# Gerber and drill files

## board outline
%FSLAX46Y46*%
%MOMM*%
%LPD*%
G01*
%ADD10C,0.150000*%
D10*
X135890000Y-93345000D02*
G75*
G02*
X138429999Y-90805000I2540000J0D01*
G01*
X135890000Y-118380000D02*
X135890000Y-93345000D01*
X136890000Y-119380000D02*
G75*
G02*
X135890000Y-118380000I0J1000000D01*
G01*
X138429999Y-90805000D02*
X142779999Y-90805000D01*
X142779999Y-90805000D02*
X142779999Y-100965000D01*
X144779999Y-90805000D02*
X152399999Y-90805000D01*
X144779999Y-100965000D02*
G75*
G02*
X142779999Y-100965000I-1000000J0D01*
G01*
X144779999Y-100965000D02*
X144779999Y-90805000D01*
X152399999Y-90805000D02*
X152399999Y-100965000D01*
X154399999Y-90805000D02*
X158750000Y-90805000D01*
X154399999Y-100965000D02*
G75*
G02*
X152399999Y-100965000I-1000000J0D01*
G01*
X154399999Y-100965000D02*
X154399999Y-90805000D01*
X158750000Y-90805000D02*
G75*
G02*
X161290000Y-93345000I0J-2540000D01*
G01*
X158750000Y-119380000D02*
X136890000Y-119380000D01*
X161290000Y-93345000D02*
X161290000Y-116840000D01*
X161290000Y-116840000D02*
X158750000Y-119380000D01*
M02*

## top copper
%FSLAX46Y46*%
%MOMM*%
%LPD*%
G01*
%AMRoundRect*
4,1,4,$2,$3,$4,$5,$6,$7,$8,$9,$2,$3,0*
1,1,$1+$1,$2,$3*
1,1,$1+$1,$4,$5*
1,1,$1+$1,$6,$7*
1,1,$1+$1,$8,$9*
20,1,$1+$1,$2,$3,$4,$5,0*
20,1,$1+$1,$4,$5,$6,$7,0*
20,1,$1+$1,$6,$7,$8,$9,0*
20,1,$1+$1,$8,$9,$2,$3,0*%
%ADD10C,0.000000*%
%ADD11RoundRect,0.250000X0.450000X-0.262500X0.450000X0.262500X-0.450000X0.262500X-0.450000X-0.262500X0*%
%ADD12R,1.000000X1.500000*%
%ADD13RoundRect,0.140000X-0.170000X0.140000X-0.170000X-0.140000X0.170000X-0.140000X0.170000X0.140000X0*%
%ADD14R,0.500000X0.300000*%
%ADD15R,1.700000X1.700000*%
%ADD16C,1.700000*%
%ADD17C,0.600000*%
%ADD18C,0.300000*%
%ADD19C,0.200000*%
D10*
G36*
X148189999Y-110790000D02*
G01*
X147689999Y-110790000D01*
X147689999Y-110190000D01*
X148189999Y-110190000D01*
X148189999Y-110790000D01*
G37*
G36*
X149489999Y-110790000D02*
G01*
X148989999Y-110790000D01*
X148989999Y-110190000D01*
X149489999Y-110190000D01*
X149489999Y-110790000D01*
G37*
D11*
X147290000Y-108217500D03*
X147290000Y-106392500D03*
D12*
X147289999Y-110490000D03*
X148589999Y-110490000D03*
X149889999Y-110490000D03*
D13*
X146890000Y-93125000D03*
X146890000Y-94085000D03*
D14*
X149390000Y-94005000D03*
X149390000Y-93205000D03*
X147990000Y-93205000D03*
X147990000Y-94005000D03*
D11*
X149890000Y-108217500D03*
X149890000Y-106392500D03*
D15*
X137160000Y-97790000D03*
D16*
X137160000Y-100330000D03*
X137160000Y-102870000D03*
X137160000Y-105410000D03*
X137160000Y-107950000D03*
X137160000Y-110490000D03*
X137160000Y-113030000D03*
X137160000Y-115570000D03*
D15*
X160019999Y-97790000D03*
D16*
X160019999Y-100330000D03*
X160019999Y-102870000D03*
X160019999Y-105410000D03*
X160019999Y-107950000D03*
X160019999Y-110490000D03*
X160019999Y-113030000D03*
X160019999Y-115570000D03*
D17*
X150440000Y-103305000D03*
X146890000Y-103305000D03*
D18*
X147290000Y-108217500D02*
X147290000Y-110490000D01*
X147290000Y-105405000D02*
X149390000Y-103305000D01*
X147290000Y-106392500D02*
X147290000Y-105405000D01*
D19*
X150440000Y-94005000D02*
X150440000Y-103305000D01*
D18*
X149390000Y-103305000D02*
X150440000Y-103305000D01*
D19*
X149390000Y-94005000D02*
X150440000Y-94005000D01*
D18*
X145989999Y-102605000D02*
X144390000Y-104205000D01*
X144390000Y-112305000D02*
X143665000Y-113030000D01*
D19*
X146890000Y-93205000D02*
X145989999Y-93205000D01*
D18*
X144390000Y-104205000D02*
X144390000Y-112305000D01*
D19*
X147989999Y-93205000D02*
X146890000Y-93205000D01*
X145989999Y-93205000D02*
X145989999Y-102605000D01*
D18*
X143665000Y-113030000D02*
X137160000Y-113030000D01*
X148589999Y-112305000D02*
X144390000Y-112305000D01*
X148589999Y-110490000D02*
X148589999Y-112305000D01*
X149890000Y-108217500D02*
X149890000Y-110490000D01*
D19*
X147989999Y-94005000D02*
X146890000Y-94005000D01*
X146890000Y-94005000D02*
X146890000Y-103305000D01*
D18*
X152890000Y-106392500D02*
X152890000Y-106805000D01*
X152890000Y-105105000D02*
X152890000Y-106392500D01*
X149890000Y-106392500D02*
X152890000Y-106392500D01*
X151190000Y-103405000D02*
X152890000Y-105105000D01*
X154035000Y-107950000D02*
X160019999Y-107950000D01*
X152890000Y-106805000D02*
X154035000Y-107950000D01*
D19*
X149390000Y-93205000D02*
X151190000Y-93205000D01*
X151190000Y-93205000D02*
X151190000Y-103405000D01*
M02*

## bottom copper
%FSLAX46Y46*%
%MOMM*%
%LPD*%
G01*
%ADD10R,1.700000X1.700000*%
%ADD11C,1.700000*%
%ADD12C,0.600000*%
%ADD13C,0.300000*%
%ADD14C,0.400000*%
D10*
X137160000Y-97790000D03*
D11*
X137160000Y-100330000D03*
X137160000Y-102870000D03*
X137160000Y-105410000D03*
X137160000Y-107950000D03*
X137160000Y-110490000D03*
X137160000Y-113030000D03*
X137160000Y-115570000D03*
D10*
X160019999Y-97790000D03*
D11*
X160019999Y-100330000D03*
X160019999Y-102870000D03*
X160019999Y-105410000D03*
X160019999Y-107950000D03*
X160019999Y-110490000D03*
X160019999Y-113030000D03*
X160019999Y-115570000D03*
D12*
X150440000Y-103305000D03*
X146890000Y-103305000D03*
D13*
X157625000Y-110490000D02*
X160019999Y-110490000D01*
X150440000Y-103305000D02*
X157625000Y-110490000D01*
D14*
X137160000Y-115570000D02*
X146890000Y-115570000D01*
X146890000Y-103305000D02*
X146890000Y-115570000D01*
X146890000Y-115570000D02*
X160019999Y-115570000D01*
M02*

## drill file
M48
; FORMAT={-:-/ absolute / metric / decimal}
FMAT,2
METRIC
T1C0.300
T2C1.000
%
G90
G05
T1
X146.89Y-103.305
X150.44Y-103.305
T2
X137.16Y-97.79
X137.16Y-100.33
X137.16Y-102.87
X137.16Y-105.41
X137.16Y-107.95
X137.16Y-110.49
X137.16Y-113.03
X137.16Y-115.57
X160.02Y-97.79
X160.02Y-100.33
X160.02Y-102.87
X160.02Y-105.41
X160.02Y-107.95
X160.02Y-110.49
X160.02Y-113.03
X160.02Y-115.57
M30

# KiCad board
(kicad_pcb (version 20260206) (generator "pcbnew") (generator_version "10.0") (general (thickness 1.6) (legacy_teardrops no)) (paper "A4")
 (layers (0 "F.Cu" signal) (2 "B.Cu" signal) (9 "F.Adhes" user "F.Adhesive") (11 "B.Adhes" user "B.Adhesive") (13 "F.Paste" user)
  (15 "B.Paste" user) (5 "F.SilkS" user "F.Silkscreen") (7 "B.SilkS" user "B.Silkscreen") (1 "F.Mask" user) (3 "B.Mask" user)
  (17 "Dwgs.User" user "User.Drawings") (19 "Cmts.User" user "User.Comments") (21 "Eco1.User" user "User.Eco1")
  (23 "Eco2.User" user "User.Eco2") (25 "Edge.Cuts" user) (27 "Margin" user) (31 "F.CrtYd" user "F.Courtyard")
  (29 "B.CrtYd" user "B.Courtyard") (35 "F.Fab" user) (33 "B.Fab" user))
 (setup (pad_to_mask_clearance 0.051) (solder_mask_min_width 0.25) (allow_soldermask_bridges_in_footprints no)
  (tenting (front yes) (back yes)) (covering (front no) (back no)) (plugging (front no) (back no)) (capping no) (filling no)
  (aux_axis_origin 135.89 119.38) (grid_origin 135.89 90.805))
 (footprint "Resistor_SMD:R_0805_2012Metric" (layer "F.Cu") (at 147.29 107.305 90)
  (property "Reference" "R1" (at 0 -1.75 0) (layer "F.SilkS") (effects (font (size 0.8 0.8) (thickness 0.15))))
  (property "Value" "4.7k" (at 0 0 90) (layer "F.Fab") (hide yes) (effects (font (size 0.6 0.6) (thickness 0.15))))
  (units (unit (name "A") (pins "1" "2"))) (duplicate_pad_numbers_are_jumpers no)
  (pad "1" smd roundrect (at -0.9125 0 90) (size 1.025 1.4) (layers "F.Cu" "F.Mask" "F.Paste") (roundrect_rratio 0.243902)
   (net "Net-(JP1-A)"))
  (pad "2" smd roundrect (at 0.9125 0 90) (size 1.025 1.4) (layers "F.Cu" "F.Mask" "F.Paste") (roundrect_rratio 0.243902) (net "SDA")))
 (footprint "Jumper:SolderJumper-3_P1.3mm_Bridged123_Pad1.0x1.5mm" (layer "F.Cu") (at 148.589999 110.49)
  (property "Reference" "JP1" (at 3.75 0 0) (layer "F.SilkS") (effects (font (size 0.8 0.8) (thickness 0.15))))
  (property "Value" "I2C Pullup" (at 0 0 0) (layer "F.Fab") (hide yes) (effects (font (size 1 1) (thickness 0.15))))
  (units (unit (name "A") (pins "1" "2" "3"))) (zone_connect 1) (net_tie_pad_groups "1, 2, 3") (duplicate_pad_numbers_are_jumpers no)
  (fp_poly (pts (xy -0.9 -0.3) (xy -0.4 -0.3) (xy -0.4 0.3) (xy -0.9 0.3)) (stroke (width 0) (type solid)) (fill yes) (layer "F.Cu"))
  (fp_poly (pts (xy 0.4 -0.3) (xy 0.9 -0.3) (xy 0.9 0.3) (xy 0.4 0.3)) (stroke (width 0) (type solid)) (fill yes) (layer "F.Cu"))
  (pad "1" smd rect (at -1.3 0) (size 1 1.5) (layers "F.Cu" "F.Mask") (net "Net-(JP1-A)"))
  (pad "2" smd rect (at 0 0) (size 1 1.5) (layers "F.Cu" "F.Mask") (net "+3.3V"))
  (pad "3" smd rect (at 1.3 0) (size 1 1.5) (layers "F.Cu" "F.Mask") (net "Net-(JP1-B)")))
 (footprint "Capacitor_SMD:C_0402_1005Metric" (layer "F.Cu") (at 146.89 93.605 -90)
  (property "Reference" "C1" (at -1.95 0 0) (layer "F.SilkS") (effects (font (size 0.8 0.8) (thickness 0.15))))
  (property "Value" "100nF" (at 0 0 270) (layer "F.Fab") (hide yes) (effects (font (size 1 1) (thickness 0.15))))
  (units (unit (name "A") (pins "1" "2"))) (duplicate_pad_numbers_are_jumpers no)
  (pad "1" smd roundrect (at -0.48 0 270) (size 0.56 0.62) (layers "F.Cu" "F.Mask" "F.Paste") (roundrect_rratio 0.25) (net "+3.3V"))
  (pad "2" smd roundrect (at 0.48 0 270) (size 0.56 0.62) (layers "F.Cu" "F.Mask" "F.Paste") (roundrect_rratio 0.25) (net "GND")))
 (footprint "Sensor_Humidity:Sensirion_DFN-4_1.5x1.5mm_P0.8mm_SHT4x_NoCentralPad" (layer "F.Cu") (at 148.69 93.605 180)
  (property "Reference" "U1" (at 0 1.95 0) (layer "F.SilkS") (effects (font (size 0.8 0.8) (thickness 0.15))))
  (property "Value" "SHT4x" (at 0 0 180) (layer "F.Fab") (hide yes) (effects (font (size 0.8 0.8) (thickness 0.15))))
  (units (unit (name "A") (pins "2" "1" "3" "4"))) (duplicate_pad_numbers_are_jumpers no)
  (pad "1" smd rect (at -0.7 -0.4 180) (size 0.5 0.3) (layers "F.Cu" "F.Mask" "F.Paste") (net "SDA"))
  (pad "2" smd rect (at -0.7 0.4 180) (size 0.5 0.3) (layers "F.Cu" "F.Mask" "F.Paste") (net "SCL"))
  (pad "3" smd rect (at 0.7 0.4 180) (size 0.5 0.3) (layers "F.Cu" "F.Mask" "F.Paste") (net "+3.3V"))
  (pad "4" smd rect (at 0.7 -0.4 180) (size 0.5 0.3) (layers "F.Cu" "F.Mask" "F.Paste") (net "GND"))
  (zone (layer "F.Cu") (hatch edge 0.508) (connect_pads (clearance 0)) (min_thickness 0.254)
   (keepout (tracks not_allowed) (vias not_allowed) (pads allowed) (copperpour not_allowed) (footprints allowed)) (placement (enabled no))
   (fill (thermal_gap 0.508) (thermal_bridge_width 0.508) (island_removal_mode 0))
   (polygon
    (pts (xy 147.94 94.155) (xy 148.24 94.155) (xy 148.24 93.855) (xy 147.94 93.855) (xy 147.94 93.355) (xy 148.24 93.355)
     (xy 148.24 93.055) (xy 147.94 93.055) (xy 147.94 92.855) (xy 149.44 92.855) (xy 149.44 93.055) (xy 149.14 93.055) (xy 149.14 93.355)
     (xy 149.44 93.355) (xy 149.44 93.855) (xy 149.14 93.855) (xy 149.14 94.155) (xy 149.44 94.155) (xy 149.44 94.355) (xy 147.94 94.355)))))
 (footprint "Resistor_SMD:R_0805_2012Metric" (layer "F.Cu") (at 149.89 107.305 90)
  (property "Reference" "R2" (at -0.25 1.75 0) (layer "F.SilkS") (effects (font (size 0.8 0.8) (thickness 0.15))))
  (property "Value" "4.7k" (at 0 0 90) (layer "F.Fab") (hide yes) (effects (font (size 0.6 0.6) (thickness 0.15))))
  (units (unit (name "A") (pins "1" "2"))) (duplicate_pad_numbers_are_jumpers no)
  (pad "1" smd roundrect (at -0.9125 0 90) (size 1.025 1.4) (layers "F.Cu" "F.Mask" "F.Paste") (roundrect_rratio 0.243902)
   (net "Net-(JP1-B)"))
  (pad "2" smd roundrect (at 0.9125 0 90) (size 1.025 1.4) (layers "F.Cu" "F.Mask" "F.Paste") (roundrect_rratio 0.243902) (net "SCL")))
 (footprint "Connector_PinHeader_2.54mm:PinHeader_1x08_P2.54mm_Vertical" (layer "B.Cu") (at 137.16 97.79 180)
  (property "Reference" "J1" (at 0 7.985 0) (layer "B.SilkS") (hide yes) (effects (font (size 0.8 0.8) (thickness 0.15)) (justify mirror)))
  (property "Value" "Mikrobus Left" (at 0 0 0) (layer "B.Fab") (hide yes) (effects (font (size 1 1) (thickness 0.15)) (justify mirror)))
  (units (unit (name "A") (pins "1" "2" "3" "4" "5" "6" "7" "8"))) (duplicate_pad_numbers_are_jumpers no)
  (pad "1" thru_hole rect (at 0 0 180) (size 1.7 1.7) (drill 1) (layers "*.Cu" "*.Mask") (remove_unused_layers no)
   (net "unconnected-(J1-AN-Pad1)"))
  (pad "2" thru_hole circle (at 0 -2.54 180) (size 1.7 1.7) (drill 1) (layers "*.Cu" "*.Mask") (remove_unused_layers no)
   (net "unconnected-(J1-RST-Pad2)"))
  (pad "3" thru_hole circle (at 0 -5.08 180) (size 1.7 1.7) (drill 1) (layers "*.Cu" "*.Mask") (remove_unused_layers no)
   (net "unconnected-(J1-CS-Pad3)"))
  (pad "4" thru_hole circle (at 0 -7.62 180) (size 1.7 1.7) (drill 1) (layers "*.Cu" "*.Mask") (remove_unused_layers no)
   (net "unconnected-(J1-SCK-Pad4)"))
  (pad "5" thru_hole circle (at 0 -10.16 180) (size 1.7 1.7) (drill 1) (layers "*.Cu" "*.Mask") (remove_unused_layers no)
   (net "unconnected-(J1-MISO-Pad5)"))
  (pad "6" thru_hole circle (at 0 -12.7 180) (size 1.7 1.7) (drill 1) (layers "*.Cu" "*.Mask") (remove_unused_layers no)
   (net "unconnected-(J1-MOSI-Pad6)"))
  (pad "7" thru_hole circle (at 0 -15.24 180) (size 1.7 1.7) (drill 1) (layers "*.Cu" "*.Mask") (remove_unused_layers no) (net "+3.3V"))
  (pad "8" thru_hole circle (at 0 -17.78 180) (size 1.7 1.7) (drill 1) (layers "*.Cu" "*.Mask") (remove_unused_layers no) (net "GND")))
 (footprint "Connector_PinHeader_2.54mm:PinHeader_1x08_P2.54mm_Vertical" (layer "B.Cu") (at 160.019999 97.79 180)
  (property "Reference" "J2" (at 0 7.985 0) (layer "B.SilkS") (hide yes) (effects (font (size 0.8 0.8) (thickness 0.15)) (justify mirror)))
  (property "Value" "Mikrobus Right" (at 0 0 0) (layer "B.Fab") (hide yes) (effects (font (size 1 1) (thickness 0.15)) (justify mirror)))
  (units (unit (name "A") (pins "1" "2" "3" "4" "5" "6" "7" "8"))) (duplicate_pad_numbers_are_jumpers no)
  (pad "1" thru_hole rect (at 0 0 180) (size 1.7 1.7) (drill 1) (layers "*.Cu" "*.Mask") (remove_unused_layers no)
   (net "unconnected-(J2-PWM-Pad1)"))
  (pad "2" thru_hole circle (at 0 -2.54 180) (size 1.7 1.7) (drill 1) (layers "*.Cu" "*.Mask") (remove_unused_layers no)
   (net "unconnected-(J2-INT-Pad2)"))
  (pad "3" thru_hole circle (at 0 -5.08 180) (size 1.7 1.7) (drill 1) (layers "*.Cu" "*.Mask") (remove_unused_layers no)
   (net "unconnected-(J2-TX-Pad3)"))
  (pad "4" thru_hole circle (at 0 -7.62 180) (size 1.7 1.7) (drill 1) (layers "*.Cu" "*.Mask") (remove_unused_layers no)
   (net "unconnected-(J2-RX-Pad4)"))
  (pad "5" thru_hole circle (at 0 -10.16 180) (size 1.7 1.7) (drill 1) (layers "*.Cu" "*.Mask") (remove_unused_layers no) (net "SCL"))
  (pad "6" thru_hole circle (at 0 -12.7 180) (size 1.7 1.7) (drill 1) (layers "*.Cu" "*.Mask") (remove_unused_layers no) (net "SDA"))
  (pad "7" thru_hole circle (at 0 -15.24 180) (size 1.7 1.7) (drill 1) (layers "*.Cu" "*.Mask") (remove_unused_layers no)
   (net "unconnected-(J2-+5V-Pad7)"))
  (pad "8" thru_hole circle (at 0 -17.78 180) (size 1.7 1.7) (drill 1) (layers "*.Cu" "*.Mask") (remove_unused_layers no) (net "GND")))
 (gr_arc (start 135.89 93.345) (mid 136.633948 91.548948) (end 138.429999 90.805) (stroke (width 0.15) (type default)) (layer "Edge.Cuts"))
 (gr_line (start 135.89 118.38) (end 135.89 93.345) (stroke (width 0.15) (type default)) (layer "Edge.Cuts"))
 (gr_arc (start 136.89 119.38) (mid 136.182893 119.087106) (end 135.89 118.38) (stroke (width 0.15) (type default)) (layer "Edge.Cuts"))
 (gr_line (start 138.429999 90.805) (end 142.779999 90.805) (stroke (width 0.15) (type default)) (layer "Edge.Cuts"))
 (gr_line (start 142.779999 90.805) (end 142.779999 100.965) (stroke (width 0.15) (type default)) (layer "Edge.Cuts"))
 (gr_line (start 144.779999 90.805) (end 152.399999 90.805) (stroke (width 0.15) (type default)) (layer "Edge.Cuts"))
 (gr_arc (start 144.779999 100.965) (mid 143.779999 101.965) (end 142.779999 100.965) (stroke (width 0.15) (type default))
  (layer "Edge.Cuts"))
 (gr_line (start 144.779999 100.965) (end 144.779999 90.805) (stroke (width 0.15) (type default)) (layer "Edge.Cuts"))
 (gr_line (start 152.399999 90.805) (end 152.399999 100.965) (stroke (width 0.15) (type default)) (layer "Edge.Cuts"))
 (gr_line (start 154.399999 90.805) (end 158.75 90.805) (stroke (width 0.15) (type default)) (layer "Edge.Cuts"))
 (gr_arc (start 154.399999 100.965) (mid 153.399999 101.965) (end 152.399999 100.965) (stroke (width 0.15) (type default))
  (layer "Edge.Cuts"))
 (gr_line (start 154.399999 100.965) (end 154.399999 90.805) (stroke (width 0.15) (type default)) (layer "Edge.Cuts"))
 (gr_arc (start 158.75 90.805) (mid 160.546051 91.548948) (end 161.29 93.345) (stroke (width 0.15) (type default)) (layer "Edge.Cuts"))
 (gr_line (start 158.75 119.38) (end 136.89 119.38) (stroke (width 0.15) (type default)) (layer "Edge.Cuts"))
 (gr_line (start 161.29 93.345) (end 161.29 116.84) (stroke (width 0.15) (type default)) (layer "Edge.Cuts"))
 (gr_line (start 161.29 116.84) (end 158.75 119.38) (stroke (width 0.15) (type default)) (layer "Edge.Cuts"))
 (segment (start 147.29 108.2175) (end 147.29 110.49) (width 0.3) (layer "F.Cu") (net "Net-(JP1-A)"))
 (segment (start 147.29 105.405) (end 149.39 103.305) (width 0.3) (layer "F.Cu") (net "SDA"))
 (segment (start 147.29 106.3925) (end 147.29 105.405) (width 0.3) (layer "F.Cu") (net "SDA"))
 (segment (start 150.44 94.005) (end 150.44 103.305) (width 0.2) (layer "F.Cu") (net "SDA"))
 (segment (start 149.39 103.305) (end 150.44 103.305) (width 0.3) (layer "F.Cu") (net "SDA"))
 (segment (start 149.39 94.005) (end 150.44 94.005) (width 0.2) (layer "F.Cu") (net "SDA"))
 (via (at 150.44 103.305) (size 0.6) (drill 0.3) (layers "F.Cu" "B.Cu") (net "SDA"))
 (segment (start 157.625 110.49) (end 160.019999 110.49) (width 0.3) (layer "B.Cu") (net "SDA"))
 (segment (start 150.44 103.305) (end 157.625 110.49) (width 0.3) (layer "B.Cu") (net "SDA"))
 (segment (start 145.989999 102.605) (end 144.39 104.205) (width 0.3) (layer "F.Cu") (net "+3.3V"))
 (segment (start 144.39 112.305) (end 143.665 113.03) (width 0.3) (layer "F.Cu") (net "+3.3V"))
 (segment (start 146.89 93.205) (end 145.989999 93.205) (width 0.2) (layer "F.Cu") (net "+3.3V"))
 (segment (start 144.39 104.205) (end 144.39 112.305) (width 0.3) (layer "F.Cu") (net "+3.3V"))
 (segment (start 147.989999 93.205) (end 146.89 93.205) (width 0.2) (layer "F.Cu") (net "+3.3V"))
 (segment (start 145.989999 93.205) (end 145.989999 102.605) (width 0.2) (layer "F.Cu") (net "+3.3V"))
 (segment (start 143.665 113.03) (end 137.16 113.03) (width 0.3) (layer "F.Cu") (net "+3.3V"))
 (segment (start 148.589999 112.305) (end 144.39 112.305) (width 0.3) (layer "F.Cu") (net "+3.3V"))
 (segment (start 148.589999 110.49) (end 148.589999 112.305) (width 0.3) (layer "F.Cu") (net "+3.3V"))
 (segment (start 149.89 108.2175) (end 149.89 110.49) (width 0.3) (layer "F.Cu") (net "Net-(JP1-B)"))
 (segment (start 147.989999 94.005) (end 146.89 94.005) (width 0.2) (layer "F.Cu") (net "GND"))
 (segment (start 146.89 94.005) (end 146.89 103.305) (width 0.2) (layer "F.Cu") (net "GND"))
 (via (at 146.89 103.305) (size 0.6) (drill 0.3) (layers "F.Cu" "B.Cu") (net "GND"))
 (segment (start 137.16 115.57) (end 146.89 115.57) (width 0.4) (layer "B.Cu") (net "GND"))
 (segment (start 146.89 103.305) (end 146.89 115.57) (width 0.4) (layer "B.Cu") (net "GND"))
 (segment (start 146.89 115.57) (end 160.019999 115.57) (width 0.4) (layer "B.Cu") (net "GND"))
 (segment (start 152.89 106.3925) (end 152.89 106.805) (width 0.3) (layer "F.Cu") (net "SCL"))
 (segment (start 152.89 105.105) (end 152.89 106.3925) (width 0.3) (layer "F.Cu") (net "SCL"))
 (segment (start 149.89 106.3925) (end 152.89 106.3925) (width 0.3) (layer "F.Cu") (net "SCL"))
 (segment (start 151.19 103.405) (end 152.89 105.105) (width 0.3) (layer "F.Cu") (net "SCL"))
 (segment (start 154.035 107.95) (end 160.019999 107.95) (width 0.3) (layer "F.Cu") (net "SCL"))
 (segment (start 152.89 106.805) (end 154.035 107.95) (width 0.3) (layer "F.Cu") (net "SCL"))
 (segment (start 149.39 93.205) (end 151.19 93.205) (width 0.2) (layer "F.Cu") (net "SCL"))
 (segment (start 151.19 93.205) (end 151.19 103.405) (width 0.2) (layer "F.Cu") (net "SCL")))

